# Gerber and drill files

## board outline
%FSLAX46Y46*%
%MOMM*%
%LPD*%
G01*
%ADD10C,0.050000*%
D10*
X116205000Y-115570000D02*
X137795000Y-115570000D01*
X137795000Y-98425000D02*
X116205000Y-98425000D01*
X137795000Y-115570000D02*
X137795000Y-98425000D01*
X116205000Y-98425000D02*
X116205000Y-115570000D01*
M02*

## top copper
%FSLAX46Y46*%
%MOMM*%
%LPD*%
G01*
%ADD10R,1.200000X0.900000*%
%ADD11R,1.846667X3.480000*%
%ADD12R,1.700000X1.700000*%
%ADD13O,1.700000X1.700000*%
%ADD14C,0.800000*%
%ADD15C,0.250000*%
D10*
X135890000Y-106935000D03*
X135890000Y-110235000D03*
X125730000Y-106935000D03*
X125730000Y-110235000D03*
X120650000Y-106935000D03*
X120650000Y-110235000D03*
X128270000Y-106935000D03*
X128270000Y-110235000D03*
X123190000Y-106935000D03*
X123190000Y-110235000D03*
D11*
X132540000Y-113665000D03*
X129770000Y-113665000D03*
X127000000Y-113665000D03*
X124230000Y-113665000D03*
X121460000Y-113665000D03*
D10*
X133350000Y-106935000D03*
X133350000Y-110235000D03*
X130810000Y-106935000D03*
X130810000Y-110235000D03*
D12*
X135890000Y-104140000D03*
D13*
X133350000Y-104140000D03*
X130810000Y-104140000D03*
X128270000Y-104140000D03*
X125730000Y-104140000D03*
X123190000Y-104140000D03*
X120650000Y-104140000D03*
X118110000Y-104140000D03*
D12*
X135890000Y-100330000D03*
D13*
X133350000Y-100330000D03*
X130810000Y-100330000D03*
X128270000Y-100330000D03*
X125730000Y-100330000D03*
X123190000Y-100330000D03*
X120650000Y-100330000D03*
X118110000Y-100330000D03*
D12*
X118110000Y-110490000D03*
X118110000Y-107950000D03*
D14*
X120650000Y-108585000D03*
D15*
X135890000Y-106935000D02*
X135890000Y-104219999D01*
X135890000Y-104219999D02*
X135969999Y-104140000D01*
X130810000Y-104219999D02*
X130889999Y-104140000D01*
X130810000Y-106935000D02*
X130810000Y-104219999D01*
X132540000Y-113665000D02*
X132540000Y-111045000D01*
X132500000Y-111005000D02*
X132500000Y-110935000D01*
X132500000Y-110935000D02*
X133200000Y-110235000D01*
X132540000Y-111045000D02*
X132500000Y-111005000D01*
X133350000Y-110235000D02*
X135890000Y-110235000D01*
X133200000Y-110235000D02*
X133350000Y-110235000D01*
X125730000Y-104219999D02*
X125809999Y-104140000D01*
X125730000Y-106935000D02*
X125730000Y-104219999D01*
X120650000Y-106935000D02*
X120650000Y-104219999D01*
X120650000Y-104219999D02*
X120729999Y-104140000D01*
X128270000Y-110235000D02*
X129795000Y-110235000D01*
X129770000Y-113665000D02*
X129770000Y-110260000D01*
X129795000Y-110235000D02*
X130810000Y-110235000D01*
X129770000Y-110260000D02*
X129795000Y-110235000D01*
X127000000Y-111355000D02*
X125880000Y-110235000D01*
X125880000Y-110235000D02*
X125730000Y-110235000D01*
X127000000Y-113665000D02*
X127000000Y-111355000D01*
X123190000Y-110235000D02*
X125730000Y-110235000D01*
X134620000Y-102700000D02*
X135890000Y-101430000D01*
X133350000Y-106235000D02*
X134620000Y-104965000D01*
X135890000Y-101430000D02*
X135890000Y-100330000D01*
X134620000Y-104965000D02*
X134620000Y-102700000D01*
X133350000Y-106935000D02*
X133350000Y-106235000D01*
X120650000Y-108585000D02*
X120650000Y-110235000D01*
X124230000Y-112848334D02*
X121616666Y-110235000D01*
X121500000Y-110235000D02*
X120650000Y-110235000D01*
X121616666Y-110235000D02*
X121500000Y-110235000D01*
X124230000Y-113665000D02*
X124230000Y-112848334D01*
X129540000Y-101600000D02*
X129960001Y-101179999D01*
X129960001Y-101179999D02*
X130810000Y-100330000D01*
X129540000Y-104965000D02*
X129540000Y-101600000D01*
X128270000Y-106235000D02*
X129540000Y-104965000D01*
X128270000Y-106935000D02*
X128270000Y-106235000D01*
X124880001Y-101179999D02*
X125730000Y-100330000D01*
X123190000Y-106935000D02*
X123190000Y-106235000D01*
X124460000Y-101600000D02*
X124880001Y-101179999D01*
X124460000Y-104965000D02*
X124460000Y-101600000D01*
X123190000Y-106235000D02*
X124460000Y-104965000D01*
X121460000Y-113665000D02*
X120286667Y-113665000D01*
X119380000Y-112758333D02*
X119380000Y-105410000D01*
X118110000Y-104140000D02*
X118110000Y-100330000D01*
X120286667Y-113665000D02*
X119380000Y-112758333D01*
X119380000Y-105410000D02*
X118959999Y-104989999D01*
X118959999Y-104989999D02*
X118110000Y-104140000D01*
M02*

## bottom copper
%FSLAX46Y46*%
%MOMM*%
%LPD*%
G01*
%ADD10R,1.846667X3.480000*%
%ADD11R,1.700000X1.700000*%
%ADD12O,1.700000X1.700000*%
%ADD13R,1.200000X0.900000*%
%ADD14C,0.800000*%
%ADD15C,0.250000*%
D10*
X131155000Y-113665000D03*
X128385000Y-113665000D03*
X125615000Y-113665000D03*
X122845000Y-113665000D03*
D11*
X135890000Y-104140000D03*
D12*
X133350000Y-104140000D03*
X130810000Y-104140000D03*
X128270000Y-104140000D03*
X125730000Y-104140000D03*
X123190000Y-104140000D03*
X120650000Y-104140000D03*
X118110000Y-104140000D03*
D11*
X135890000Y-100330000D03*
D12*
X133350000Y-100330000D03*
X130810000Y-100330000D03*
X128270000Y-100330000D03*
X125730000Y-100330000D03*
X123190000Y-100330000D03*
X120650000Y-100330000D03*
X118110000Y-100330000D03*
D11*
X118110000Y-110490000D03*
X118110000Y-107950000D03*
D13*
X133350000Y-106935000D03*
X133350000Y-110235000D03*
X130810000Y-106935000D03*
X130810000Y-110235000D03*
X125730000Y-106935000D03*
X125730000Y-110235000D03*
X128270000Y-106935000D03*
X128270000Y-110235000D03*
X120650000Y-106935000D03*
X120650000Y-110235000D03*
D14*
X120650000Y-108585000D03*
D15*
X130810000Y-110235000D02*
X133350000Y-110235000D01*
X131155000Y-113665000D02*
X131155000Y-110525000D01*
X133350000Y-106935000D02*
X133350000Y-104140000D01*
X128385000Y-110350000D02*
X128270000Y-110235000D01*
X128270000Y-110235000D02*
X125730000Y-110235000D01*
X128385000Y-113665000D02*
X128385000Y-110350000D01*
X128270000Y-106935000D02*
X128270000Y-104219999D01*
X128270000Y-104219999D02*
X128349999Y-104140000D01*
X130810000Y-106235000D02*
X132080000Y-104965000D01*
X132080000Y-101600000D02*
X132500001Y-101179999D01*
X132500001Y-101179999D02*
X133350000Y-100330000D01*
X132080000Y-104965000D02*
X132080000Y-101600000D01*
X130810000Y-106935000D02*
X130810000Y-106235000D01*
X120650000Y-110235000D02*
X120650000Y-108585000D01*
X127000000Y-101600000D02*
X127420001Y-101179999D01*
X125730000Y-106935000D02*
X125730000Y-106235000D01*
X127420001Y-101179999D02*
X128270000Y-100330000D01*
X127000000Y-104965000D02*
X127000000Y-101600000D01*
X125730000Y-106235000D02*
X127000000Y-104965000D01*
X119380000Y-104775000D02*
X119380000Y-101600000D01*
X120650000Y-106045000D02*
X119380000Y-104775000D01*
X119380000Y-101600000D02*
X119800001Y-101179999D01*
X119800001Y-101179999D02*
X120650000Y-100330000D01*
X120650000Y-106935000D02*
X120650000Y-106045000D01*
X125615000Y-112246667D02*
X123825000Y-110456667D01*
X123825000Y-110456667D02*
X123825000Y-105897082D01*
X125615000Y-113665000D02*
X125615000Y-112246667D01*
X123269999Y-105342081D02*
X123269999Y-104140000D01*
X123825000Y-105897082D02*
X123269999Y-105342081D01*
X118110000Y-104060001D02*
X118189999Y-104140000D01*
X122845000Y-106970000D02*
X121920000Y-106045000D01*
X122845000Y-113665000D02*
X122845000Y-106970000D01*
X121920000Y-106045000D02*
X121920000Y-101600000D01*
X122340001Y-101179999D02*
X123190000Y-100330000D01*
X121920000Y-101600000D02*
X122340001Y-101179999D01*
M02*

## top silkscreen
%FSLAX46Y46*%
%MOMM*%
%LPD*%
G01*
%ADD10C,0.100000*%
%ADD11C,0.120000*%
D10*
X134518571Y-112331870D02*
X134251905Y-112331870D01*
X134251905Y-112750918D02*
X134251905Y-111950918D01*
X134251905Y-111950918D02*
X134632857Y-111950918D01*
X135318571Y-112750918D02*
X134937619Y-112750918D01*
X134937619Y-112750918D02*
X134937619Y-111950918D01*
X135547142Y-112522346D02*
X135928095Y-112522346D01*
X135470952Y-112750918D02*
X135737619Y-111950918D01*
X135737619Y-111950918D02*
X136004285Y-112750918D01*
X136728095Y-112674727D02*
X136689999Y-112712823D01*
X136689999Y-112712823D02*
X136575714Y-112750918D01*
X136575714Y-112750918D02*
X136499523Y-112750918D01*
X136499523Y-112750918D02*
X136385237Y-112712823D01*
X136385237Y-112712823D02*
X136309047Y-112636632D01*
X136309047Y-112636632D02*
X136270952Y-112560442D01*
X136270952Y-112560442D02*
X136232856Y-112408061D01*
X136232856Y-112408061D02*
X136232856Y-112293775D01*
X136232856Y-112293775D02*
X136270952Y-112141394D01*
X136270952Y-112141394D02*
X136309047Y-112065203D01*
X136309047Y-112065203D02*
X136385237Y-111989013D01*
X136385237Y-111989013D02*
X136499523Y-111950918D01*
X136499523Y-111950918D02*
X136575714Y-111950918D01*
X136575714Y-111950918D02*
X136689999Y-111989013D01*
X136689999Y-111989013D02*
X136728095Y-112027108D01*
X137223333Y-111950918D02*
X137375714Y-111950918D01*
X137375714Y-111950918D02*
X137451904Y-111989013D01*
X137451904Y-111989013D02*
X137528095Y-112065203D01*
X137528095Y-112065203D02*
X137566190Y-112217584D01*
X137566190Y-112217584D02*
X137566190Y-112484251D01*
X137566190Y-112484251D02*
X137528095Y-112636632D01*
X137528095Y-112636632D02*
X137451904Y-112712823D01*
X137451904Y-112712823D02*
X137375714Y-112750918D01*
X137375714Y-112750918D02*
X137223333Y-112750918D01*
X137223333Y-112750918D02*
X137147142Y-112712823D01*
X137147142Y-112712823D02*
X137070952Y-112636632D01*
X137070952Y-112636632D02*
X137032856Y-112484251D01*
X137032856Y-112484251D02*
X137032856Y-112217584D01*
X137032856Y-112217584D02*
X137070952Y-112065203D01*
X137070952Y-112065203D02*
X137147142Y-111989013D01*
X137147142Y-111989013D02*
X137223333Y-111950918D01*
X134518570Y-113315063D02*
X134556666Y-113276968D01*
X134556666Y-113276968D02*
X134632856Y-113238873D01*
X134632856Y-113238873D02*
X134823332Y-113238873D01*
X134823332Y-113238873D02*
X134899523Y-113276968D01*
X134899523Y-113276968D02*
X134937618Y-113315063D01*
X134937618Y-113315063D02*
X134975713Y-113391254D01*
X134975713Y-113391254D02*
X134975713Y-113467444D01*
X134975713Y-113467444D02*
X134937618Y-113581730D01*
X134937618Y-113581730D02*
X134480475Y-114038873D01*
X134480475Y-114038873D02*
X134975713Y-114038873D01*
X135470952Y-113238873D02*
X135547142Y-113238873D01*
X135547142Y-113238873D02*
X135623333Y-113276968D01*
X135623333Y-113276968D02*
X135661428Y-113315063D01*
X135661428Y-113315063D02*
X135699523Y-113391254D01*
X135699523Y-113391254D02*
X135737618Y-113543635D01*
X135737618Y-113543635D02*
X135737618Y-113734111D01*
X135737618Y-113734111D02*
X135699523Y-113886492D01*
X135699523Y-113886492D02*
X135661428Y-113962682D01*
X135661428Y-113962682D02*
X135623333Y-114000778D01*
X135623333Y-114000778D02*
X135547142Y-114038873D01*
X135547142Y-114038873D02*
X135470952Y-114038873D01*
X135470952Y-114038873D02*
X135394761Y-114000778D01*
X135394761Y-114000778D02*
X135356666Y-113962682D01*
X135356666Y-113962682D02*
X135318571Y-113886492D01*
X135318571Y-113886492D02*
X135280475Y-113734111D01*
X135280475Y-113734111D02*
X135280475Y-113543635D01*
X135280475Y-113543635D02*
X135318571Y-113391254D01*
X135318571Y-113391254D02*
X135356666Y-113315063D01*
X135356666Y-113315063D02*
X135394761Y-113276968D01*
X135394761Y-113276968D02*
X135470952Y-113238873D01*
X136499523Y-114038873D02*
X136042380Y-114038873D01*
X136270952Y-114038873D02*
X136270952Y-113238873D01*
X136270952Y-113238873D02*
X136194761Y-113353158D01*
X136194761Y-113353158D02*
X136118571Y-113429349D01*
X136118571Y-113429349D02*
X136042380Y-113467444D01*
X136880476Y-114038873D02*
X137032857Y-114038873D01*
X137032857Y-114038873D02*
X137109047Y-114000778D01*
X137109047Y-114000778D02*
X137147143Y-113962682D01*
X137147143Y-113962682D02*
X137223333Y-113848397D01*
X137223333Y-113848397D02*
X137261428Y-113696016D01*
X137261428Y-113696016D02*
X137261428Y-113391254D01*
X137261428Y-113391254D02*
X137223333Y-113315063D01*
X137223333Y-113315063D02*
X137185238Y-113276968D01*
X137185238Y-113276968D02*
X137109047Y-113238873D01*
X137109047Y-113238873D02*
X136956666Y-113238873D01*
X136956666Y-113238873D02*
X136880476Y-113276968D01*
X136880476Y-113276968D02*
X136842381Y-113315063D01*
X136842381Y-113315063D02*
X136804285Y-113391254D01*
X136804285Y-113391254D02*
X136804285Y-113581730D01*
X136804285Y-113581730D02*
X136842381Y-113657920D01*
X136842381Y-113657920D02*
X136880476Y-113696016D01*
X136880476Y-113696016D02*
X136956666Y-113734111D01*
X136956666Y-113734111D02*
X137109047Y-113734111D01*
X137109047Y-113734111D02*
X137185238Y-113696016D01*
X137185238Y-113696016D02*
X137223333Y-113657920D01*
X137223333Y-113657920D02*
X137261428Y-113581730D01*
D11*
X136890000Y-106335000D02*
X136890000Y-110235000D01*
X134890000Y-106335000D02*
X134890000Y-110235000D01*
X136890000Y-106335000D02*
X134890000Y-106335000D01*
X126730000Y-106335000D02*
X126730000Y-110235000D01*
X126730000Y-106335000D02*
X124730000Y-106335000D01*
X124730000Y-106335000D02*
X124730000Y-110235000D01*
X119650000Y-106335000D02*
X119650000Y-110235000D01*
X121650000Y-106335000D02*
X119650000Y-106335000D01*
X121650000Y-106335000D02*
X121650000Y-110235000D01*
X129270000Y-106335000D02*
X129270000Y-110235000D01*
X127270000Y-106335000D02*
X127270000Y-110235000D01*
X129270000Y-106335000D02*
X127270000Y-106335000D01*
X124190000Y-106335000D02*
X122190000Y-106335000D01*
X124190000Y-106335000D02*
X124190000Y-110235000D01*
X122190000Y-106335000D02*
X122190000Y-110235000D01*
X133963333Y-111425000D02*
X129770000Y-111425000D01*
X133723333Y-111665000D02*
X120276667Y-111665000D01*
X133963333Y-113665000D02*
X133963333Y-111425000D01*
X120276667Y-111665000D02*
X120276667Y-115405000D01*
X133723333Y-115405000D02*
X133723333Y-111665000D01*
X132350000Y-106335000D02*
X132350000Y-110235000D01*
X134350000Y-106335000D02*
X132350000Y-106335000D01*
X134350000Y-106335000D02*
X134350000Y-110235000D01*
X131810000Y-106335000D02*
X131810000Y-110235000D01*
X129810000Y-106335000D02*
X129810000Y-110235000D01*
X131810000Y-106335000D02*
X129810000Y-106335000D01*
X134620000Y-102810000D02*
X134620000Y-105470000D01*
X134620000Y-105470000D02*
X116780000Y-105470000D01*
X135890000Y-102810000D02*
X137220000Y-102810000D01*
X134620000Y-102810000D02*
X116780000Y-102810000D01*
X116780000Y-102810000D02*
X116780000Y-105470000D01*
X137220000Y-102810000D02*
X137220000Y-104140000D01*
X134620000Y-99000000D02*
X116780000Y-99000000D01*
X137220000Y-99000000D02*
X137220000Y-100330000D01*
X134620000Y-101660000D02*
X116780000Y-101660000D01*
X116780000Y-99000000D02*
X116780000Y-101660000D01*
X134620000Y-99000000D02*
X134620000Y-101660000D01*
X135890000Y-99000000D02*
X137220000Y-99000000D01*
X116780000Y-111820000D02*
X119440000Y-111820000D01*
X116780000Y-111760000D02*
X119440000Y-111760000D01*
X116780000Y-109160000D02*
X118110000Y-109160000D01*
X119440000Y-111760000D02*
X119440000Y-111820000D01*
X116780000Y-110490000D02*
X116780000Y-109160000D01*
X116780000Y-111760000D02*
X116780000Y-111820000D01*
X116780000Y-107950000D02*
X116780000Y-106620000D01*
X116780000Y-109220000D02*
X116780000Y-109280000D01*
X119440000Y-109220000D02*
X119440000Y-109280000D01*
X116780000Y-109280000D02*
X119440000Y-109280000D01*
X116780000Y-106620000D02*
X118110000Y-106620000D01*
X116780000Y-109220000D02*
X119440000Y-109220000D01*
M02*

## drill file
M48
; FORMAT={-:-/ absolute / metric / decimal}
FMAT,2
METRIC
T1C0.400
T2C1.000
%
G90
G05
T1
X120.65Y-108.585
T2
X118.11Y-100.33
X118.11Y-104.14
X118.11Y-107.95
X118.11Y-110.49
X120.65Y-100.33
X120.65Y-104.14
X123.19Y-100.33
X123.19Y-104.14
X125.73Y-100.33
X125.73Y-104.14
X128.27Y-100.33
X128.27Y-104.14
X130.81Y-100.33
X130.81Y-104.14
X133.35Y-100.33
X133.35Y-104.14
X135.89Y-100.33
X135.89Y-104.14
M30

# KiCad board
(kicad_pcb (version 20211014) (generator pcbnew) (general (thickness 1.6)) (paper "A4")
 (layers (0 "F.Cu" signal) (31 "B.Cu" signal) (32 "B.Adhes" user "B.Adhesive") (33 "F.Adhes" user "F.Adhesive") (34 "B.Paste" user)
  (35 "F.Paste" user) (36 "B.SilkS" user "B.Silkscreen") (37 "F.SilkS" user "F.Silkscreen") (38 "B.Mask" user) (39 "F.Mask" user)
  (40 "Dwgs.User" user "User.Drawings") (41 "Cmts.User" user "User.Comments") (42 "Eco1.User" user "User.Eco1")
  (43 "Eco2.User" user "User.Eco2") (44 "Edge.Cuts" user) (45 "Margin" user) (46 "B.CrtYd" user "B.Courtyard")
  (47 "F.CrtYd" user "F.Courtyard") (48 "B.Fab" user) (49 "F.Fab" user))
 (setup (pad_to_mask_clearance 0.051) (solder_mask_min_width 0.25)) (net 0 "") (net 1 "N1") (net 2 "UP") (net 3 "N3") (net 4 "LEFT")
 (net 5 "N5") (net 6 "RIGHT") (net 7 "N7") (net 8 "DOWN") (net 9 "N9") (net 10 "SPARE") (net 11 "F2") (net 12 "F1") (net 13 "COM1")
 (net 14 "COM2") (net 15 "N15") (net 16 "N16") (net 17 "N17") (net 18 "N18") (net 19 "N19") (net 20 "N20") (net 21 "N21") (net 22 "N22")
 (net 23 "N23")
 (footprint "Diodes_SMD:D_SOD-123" (layer "F.Cu") (at 135.89 108.585 -90) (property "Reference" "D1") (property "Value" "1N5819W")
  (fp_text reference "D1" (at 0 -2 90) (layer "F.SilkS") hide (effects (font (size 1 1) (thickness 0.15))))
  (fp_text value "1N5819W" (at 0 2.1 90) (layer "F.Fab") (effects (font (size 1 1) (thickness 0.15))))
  (fp_line (start -2.25 -1) (end 1.65 -1) (layer "F.SilkS") (width 0.12))
  (fp_line (start -2.25 1) (end 1.65 1) (layer "F.SilkS") (width 0.12))
  (fp_line (start -2.25 -1) (end -2.25 1) (layer "F.SilkS") (width 0.12))
  (pad "1" smd rect locked (at -1.65 0 270) (size 0.9 1.2) (layers "F.Cu" "F.Paste" "F.Mask") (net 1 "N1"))
  (pad "2" smd rect locked (at 1.65 0 270) (size 0.9 1.2) (layers "F.Cu" "F.Paste" "F.Mask") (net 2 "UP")))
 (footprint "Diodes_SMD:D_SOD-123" (layer "F.Cu") (at 125.73 108.585 -90) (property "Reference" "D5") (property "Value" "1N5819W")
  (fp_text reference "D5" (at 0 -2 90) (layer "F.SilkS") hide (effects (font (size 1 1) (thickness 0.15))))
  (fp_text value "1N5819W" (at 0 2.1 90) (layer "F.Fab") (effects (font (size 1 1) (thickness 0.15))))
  (fp_line (start -2.25 -1) (end 1.65 -1) (layer "F.SilkS") (width 0.12))
  (fp_line (start -2.25 -1) (end -2.25 1) (layer "F.SilkS") (width 0.12))
  (fp_line (start -2.25 1) (end 1.65 1) (layer "F.SilkS") (width 0.12))
  (pad "1" smd rect locked (at -1.65 0 270) (size 0.9 1.2) (layers "F.Cu" "F.Paste" "F.Mask") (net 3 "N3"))
  (pad "2" smd rect locked (at 1.65 0 270) (size 0.9 1.2) (layers "F.Cu" "F.Paste" "F.Mask") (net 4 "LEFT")))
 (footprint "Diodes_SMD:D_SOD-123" (layer "F.Cu") (at 120.65 108.585 -90) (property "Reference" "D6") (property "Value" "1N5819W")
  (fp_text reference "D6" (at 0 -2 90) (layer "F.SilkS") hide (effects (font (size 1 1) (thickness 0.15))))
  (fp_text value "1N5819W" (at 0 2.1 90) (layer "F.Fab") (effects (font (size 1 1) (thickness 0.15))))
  (fp_line (start -2.25 1) (end 1.65 1) (layer "F.SilkS") (width 0.12))
  (fp_line (start -2.25 -1) (end -2.25 1) (layer "F.SilkS") (width 0.12))
  (fp_line (start -2.25 -1) (end 1.65 -1) (layer "F.SilkS") (width 0.12))
  (pad "1" smd rect locked (at -1.65 0 270) (size 0.9 1.2) (layers "F.Cu" "F.Paste" "F.Mask") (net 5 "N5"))
  (pad "2" smd rect locked (at 1.65 0 270) (size 0.9 1.2) (layers "F.Cu" "F.Paste" "F.Mask") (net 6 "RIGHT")))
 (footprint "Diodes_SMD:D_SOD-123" (layer "F.Cu") (at 128.27 108.585 -90) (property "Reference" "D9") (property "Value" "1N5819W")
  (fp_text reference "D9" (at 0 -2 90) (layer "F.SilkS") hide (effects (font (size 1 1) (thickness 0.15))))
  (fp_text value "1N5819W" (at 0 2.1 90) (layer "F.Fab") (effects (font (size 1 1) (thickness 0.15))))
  (fp_line (start -2.25 -1) (end 1.65 -1) (layer "F.SilkS") (width 0.12))
  (fp_line (start -2.25 1) (end 1.65 1) (layer "F.SilkS") (width 0.12))
  (fp_line (start -2.25 -1) (end -2.25 1) (layer "F.SilkS") (width 0.12))
  (pad "1" smd rect locked (at -1.65 0 270) (size 0.9 1.2) (layers "F.Cu" "F.Paste" "F.Mask") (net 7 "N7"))
  (pad "2" smd rect locked (at 1.65 0 270) (size 0.9 1.2) (layers "F.Cu" "F.Paste" "F.Mask") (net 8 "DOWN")))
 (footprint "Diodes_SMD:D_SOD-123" (layer "F.Cu") (at 123.19 108.585 -90) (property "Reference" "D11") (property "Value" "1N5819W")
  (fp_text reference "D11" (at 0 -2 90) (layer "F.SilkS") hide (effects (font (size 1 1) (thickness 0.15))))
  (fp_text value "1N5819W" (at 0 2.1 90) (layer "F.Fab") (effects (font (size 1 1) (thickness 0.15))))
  (fp_line (start -2.25 -1) (end -2.25 1) (layer "F.SilkS") (width 0.12))
  (fp_line (start -2.25 -1) (end 1.65 -1) (layer "F.SilkS") (width 0.12))
  (fp_line (start -2.25 1) (end 1.65 1) (layer "F.SilkS") (width 0.12))
  (pad "1" smd rect locked (at -1.65 0 270) (size 0.9 1.2) (layers "F.Cu" "F.Paste" "F.Mask") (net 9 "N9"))
  (pad "2" smd rect locked (at 1.65 0 270) (size 0.9 1.2) (layers "F.Cu" "F.Paste" "F.Mask") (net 4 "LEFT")))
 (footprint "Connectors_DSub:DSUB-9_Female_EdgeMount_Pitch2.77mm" (layer "F.Cu") (at 127 113.665) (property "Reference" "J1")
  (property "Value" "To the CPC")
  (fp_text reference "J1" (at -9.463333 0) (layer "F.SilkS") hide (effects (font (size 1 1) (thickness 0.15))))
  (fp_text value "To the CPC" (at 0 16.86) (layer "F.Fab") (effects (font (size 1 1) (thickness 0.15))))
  (fp_line (start 6.963333 -2.24) (end 2.77 -2.24) (layer "F.SilkS") (width 0.12))
  (fp_line (start 6.723333 -2) (end -6.723333 -2) (layer "F.SilkS") (width 0.12))
  (fp_line (start 6.963333 0) (end 6.963333 -2.24) (layer "F.SilkS") (width 0.12))
  (fp_line (start -6.723333 -2) (end -6.723333 1.74) (layer "F.SilkS") (width 0.12))
  (fp_line (start 6.723333 1.74) (end 6.723333 -2) (layer "F.SilkS") (width 0.12))
  (pad "1" smd rect locked (at 5.54 0) (size 1.846667 3.48) (layers "F.Cu" "F.Paste" "F.Mask") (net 2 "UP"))
  (pad "2" smd rect locked (at 2.77 0) (size 1.846667 3.48) (layers "F.Cu" "F.Paste" "F.Mask") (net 8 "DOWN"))
  (pad "3" smd rect locked (at 0 0) (size 1.846667 3.48) (layers "F.Cu" "F.Paste" "F.Mask") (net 4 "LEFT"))
  (pad "4" smd rect locked (at -2.77 0) (size 1.846667 3.48) (layers "F.Cu" "F.Paste" "F.Mask") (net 6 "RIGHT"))
  (pad "5" smd rect locked (at -5.54 0) (size 1.846667 3.48) (layers "F.Cu" "F.Paste" "F.Mask") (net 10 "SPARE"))
  (pad "6" smd rect locked (at 4.155 0) (size 1.846667 3.48) (layers "B.Cu" "B.Paste" "B.Mask") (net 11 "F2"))
  (pad "7" smd rect locked (at 1.385 0) (size 1.846667 3.48) (layers "B.Cu" "B.Paste" "B.Mask") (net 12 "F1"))
  (pad "8" smd rect locked (at -1.385 0) (size 1.846667 3.48) (layers "B.Cu" "B.Paste" "B.Mask") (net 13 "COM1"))
  (pad "9" smd rect locked (at -4.155 0) (size 1.846667 3.48) (layers "B.Cu" "B.Paste" "B.Mask") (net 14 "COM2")))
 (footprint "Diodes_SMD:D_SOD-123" (layer "F.Cu") (at 133.35 108.585 -90) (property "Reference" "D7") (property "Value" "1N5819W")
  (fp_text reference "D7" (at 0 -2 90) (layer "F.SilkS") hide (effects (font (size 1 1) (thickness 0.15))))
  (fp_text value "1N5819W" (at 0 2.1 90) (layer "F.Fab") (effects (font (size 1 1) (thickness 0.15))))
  (fp_line (start -2.25 1) (end 1.65 1) (layer "F.SilkS") (width 0.12))
  (fp_line (start -2.25 -1) (end -2.25 1) (layer "F.SilkS") (width 0.12))
  (fp_line (start -2.25 -1) (end 1.65 -1) (layer "F.SilkS") (width 0.12))
  (pad "1" smd rect locked (at -1.65 0 270) (size 0.9 1.2) (layers "F.Cu" "F.Paste" "F.Mask") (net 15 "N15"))
  (pad "2" smd rect locked (at 1.65 0 270) (size 0.9 1.2) (layers "F.Cu" "F.Paste" "F.Mask") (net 2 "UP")))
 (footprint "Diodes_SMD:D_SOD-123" (layer "F.Cu") (at 130.81 108.585 -90) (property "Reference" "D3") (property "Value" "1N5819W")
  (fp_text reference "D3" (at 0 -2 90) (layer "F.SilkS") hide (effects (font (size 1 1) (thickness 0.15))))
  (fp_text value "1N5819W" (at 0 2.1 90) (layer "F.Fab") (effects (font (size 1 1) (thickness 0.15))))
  (fp_line (start -2.25 -1) (end 1.65 -1) (layer "F.SilkS") (width 0.12))
  (fp_line (start -2.25 1) (end 1.65 1) (layer "F.SilkS") (width 0.12))
  (fp_line (start -2.25 -1) (end -2.25 1) (layer "F.SilkS") (width 0.12))
  (pad "1" smd rect locked (at -1.65 0 270) (size 0.9 1.2) (layers "F.Cu" "F.Paste" "F.Mask") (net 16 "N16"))
  (pad "2" smd rect locked (at 1.65 0 270) (size 0.9 1.2) (layers "F.Cu" "F.Paste" "F.Mask") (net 8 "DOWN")))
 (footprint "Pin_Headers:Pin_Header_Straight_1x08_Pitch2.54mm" (layer "F.Cu") (at 135.89 104.14 -90) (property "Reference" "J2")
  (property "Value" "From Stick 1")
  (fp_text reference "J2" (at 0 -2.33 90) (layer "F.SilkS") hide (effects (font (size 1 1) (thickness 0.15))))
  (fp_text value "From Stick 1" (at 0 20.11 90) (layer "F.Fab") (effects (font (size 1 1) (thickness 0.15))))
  (fp_line (start -1.33 1.27) (end 1.33 1.27) (layer "F.SilkS") (width 0.12))
  (fp_line (start 1.33 1.27) (end 1.33 19.11) (layer "F.SilkS") (width 0.12))
  (fp_line (start -1.33 0) (end -1.33 -1.33) (layer "F.SilkS") (width 0.12))
  (fp_line (start -1.33 1.27) (end -1.33 19.11) (layer "F.SilkS") (width 0.12))
  (fp_line (start -1.33 19.11) (end 1.33 19.11) (layer "F.SilkS") (width 0.12))
  (fp_line (start -1.33 -1.33) (end 0 -1.33) (layer "F.SilkS") (width 0.12))
  (pad "1" thru_hole rect locked (at 0 0 270) (size 1.7 1.7) (drill 1) (layers *.Cu *.Mask) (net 1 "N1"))
  (pad "2" thru_hole oval locked (at 0 2.54 270) (size 1.7 1.7) (drill 1) (layers *.Cu *.Mask) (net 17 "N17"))
  (pad "3" thru_hole oval locked (at 0 5.08 270) (size 1.7 1.7) (drill 1) (layers *.Cu *.Mask) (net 16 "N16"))
  (pad "4" thru_hole oval locked (at 0 7.62 270) (size 1.7 1.7) (drill 1) (layers *.Cu *.Mask) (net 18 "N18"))
  (pad "5" thru_hole oval locked (at 0 10.16 270) (size 1.7 1.7) (drill 1) (layers *.Cu *.Mask) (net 3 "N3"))
  (pad "6" thru_hole oval locked (at 0 12.7 270) (size 1.7 1.7) (drill 1) (layers *.Cu *.Mask) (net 13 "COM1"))
  (pad "7" thru_hole oval locked (at 0 15.24 270) (size 1.7 1.7) (drill 1) (layers *.Cu *.Mask) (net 5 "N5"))
  (pad "8" thru_hole oval locked (at 0 17.78 270) (size 1.7 1.7) (drill 1) (layers *.Cu *.Mask) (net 10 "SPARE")))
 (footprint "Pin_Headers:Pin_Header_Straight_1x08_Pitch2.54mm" (layer "F.Cu") (at 135.89 100.33 -90) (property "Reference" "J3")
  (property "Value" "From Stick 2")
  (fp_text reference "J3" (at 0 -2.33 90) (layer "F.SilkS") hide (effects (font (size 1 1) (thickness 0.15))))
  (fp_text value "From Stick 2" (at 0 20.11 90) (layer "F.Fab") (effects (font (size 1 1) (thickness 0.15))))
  (fp_line (start -1.33 1.27) (end -1.33 19.11) (layer "F.SilkS") (width 0.12))
  (fp_line (start -1.33 -1.33) (end 0 -1.33) (layer "F.SilkS") (width 0.12))
  (fp_line (start 1.33 1.27) (end 1.33 19.11) (layer "F.SilkS") (width 0.12))
  (fp_line (start -1.33 19.11) (end 1.33 19.11) (layer "F.SilkS") (width 0.12))
  (fp_line (start -1.33 1.27) (end 1.33 1.27) (layer "F.SilkS") (width 0.12))
  (fp_line (start -1.33 0) (end -1.33 -1.33) (layer "F.SilkS") (width 0.12))
  (pad "1" thru_hole rect locked (at 0 0 270) (size 1.7 1.7) (drill 1) (layers *.Cu *.Mask) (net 15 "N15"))
  (pad "2" thru_hole oval locked (at 0 2.54 270) (size 1.7 1.7) (drill 1) (layers *.Cu *.Mask) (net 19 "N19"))
  (pad "3" thru_hole oval locked (at 0 5.08 270) (size 1.7 1.7) (drill 1) (layers *.Cu *.Mask) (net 7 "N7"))
  (pad "4" thru_hole oval locked (at 0 7.62 270) (size 1.7 1.7) (drill 1) (layers *.Cu *.Mask) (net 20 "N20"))
  (pad "5" thru_hole oval locked (at 0 10.16 270) (size 1.7 1.7) (drill 1) (layers *.Cu *.Mask) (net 9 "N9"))
  (pad "6" thru_hole oval locked (at 0 12.7 270) (size 1.7 1.7) (drill 1) (layers *.Cu *.Mask) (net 14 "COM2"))
  (pad "7" thru_hole oval locked (at 0 15.24 270) (size 1.7 1.7) (drill 1) (layers *.Cu *.Mask) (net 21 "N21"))
  (pad "8" thru_hole oval locked (at 0 17.78 270) (size 1.7 1.7) (drill 1) (layers *.Cu *.Mask) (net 10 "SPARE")))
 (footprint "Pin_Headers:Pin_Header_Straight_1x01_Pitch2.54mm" (layer "F.Cu") (at 118.11 110.49) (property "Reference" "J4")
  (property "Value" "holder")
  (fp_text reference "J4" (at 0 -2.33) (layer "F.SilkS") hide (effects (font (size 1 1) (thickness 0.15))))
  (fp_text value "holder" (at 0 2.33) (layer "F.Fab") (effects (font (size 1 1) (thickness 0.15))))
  (fp_line (start -1.33 1.33) (end 1.33 1.33) (layer "F.SilkS") (width 0.12))
  (fp_line (start -1.33 1.27) (end 1.33 1.27) (layer "F.SilkS") (width 0.12))
  (fp_line (start -1.33 -1.33) (end 0 -1.33) (layer "F.SilkS") (width 0.12))
  (fp_line (start 1.33 1.27) (end 1.33 1.33) (layer "F.SilkS") (width 0.12))
  (fp_line (start -1.33 0) (end -1.33 -1.33) (layer "F.SilkS") (width 0.12))
  (fp_line (start -1.33 1.27) (end -1.33 1.33) (layer "F.SilkS") (width 0.12))
  (pad "1" thru_hole rect locked (at 0 0) (size 1.7 1.7) (drill 1) (layers *.Cu *.Mask) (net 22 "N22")))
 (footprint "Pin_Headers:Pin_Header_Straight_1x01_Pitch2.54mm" (layer "F.Cu") (at 118.11 107.95) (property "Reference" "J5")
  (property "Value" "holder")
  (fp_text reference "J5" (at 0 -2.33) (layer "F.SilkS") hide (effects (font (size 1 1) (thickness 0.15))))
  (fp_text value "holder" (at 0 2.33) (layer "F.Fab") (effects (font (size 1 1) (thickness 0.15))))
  (fp_line (start -1.33 0) (end -1.33 -1.33) (layer "F.SilkS") (width 0.12))
  (fp_line (start -1.33 1.27) (end -1.33 1.33) (layer "F.SilkS") (width 0.12))
  (fp_line (start 1.33 1.27) (end 1.33 1.33) (layer "F.SilkS") (width 0.12))
  (fp_line (start -1.33 1.33) (end 1.33 1.33) (layer "F.SilkS") (width 0.12))
  (fp_line (start -1.33 -1.33) (end 0 -1.33) (layer "F.SilkS") (width 0.12))
  (fp_line (start -1.33 1.27) (end 1.33 1.27) (layer "F.SilkS") (width 0.12))
  (pad "1" thru_hole rect locked (at 0 0) (size 1.7 1.7) (drill 1) (layers *.Cu *.Mask) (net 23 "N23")))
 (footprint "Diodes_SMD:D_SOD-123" (layer "B.Cu") (at 133.35 108.585 -90) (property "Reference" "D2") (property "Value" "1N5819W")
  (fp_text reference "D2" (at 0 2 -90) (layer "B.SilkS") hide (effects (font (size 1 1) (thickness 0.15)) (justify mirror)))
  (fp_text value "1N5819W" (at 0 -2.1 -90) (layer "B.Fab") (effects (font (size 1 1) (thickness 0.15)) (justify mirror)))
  (pad "1" smd rect locked (at -1.65 0 270) (size 0.9 1.2) (layers "B.Cu" "B.Paste" "B.Mask") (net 17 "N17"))
  (pad "2" smd rect locked (at 1.65 0 270) (size 0.9 1.2) (layers "B.Cu" "B.Paste" "B.Mask") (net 11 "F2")))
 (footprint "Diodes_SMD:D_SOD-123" (layer "B.Cu") (at 130.81 108.585 -90) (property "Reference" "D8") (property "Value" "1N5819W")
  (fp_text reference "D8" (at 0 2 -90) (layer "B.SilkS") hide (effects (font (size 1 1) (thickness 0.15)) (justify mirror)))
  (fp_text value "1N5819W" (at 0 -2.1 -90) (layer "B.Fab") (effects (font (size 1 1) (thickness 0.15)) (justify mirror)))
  (pad "1" smd rect locked (at -1.65 0 270) (size 0.9 1.2) (layers "B.Cu" "B.Paste" "B.Mask") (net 19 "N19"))
  (pad "2" smd rect locked (at 1.65 0 270) (size 0.9 1.2) (layers "B.Cu" "B.Paste" "B.Mask") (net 11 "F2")))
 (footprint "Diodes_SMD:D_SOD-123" (layer "B.Cu") (at 125.73 108.585 -90) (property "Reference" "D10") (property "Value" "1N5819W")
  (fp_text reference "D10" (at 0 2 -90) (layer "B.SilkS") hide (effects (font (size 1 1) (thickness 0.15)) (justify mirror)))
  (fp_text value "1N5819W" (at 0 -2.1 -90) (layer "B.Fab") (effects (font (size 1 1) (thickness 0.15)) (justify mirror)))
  (pad "1" smd rect locked (at -1.65 0 270) (size 0.9 1.2) (layers "B.Cu" "B.Paste" "B.Mask") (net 20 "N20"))
  (pad "2" smd rect locked (at 1.65 0 270) (size 0.9 1.2) (layers "B.Cu" "B.Paste" "B.Mask") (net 12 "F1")))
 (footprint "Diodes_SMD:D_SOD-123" (layer "B.Cu") (at 128.27 108.585 -90) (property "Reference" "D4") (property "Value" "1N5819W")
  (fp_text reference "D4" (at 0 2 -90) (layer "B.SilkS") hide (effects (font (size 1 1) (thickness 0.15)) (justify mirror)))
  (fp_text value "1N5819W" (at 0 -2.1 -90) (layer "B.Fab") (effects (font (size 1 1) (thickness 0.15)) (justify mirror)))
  (pad "1" smd rect locked (at -1.65 0 270) (size 0.9 1.2) (layers "B.Cu" "B.Paste" "B.Mask") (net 18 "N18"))
  (pad "2" smd rect locked (at 1.65 0 270) (size 0.9 1.2) (layers "B.Cu" "B.Paste" "B.Mask") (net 12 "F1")))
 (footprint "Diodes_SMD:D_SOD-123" (layer "B.Cu") (at 120.65 108.585 -90) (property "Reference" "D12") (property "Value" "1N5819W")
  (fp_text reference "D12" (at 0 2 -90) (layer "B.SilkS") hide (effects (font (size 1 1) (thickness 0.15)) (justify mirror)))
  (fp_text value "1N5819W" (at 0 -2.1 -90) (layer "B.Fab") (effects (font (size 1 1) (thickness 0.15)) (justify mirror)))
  (pad "1" smd rect locked (at -1.65 0 270) (size 0.9 1.2) (layers "B.Cu" "B.Paste" "B.Mask") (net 21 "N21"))
  (pad "2" smd rect locked (at 1.65 0 270) (size 0.9 1.2) (layers "B.Cu" "B.Paste" "B.Mask") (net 6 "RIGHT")))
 (gr_line (start 116.205 115.57) (end 137.795 115.57) (layer "Edge.Cuts") (width 0.05))
 (gr_line (start 137.795 98.425) (end 116.205 98.425) (layer "Edge.Cuts") (width 0.05))
 (gr_line (start 137.795 115.57) (end 137.795 98.425) (layer "Edge.Cuts") (width 0.05))
 (gr_line (start 116.205 98.425) (end 116.205 115.57) (layer "Edge.Cuts") (width 0.05))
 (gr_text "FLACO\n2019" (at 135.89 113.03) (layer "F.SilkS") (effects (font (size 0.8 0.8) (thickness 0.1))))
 (segment (start 130.81 110.235) (end 133.35 110.235) (width 0.25) (layer "B.Cu") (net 11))
 (segment (start 131.155 113.665) (end 131.155 110.525) (width 0.25) (layer "B.Cu") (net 11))
 (segment (start 135.89 106.935) (end 135.89 104.219999) (width 0.25) (layer "F.Cu") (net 1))
 (segment (start 135.89 104.219999) (end 135.969999 104.14) (width 0.25) (layer "F.Cu") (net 1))
 (segment (start 133.35 106.935) (end 133.35 104.14) (width 0.25) (layer "B.Cu") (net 17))
 (segment (start 128.385 110.35) (end 128.27 110.235) (width 0.25) (layer "B.Cu") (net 12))
 (segment (start 128.27 110.235) (end 125.73 110.235) (width 0.25) (layer "B.Cu") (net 12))
 (segment (start 128.385 113.665) (end 128.385 110.35) (width 0.25) (layer "B.Cu") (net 12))
 (segment (start 130.81 104.219999) (end 130.889999 104.14) (width 0.25) (layer "F.Cu") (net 16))
 (segment (start 130.81 106.935) (end 130.81 104.219999) (width 0.25) (layer "F.Cu") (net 16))
 (segment (start 128.27 106.935) (end 128.27 104.219999) (width 0.25) (layer "B.Cu") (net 18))
 (segment (start 128.27 104.219999) (end 128.349999 104.14) (width 0.25) (layer "B.Cu") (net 18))
 (segment (start 132.54 113.665) (end 132.54 111.045) (width 0.25) (layer "F.Cu") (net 2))
 (segment (start 132.5 111.005) (end 132.5 110.935) (width 0.25) (layer "F.Cu") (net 2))
 (segment (start 132.5 110.935) (end 133.2 110.235) (width 0.25) (layer "F.Cu") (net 2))
 (segment (start 132.54 111.045) (end 132.5 111.005) (width 0.25) (layer "F.Cu") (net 2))
 (segment (start 133.35 110.235) (end 135.89 110.235) (width 0.25) (layer "F.Cu") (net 2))
 (segment (start 133.2 110.235) (end 133.35 110.235) (width 0.25) (layer "F.Cu") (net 2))
 (segment (start 125.73 104.219999) (end 125.809999 104.14) (width 0.25) (layer "F.Cu") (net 3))
 (segment (start 125.73 106.935) (end 125.73 104.219999) (width 0.25) (layer "F.Cu") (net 3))
 (segment (start 120.65 106.935) (end 120.65 104.219999) (width 0.25) (layer "F.Cu") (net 5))
 (segment (start 120.65 104.219999) (end 120.729999 104.14) (width 0.25) (layer "F.Cu") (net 5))
 (segment (start 128.27 110.235) (end 129.795 110.235) (width 0.25) (layer "F.Cu") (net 8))
 (segment (start 129.77 113.665) (end 129.77 110.26) (width 0.25) (layer "F.Cu") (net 8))
 (segment (start 129.795 110.235) (end 130.81 110.235) (width 0.25) (layer "F.Cu") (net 8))
 (segment (start 129.77 110.26) (end 129.795 110.235) (width 0.25) (layer "F.Cu") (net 8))
 (segment (start 127 111.355) (end 125.88 110.235) (width 0.25) (layer "F.Cu") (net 4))
 (segment (start 125.88 110.235) (end 125.73 110.235) (width 0.25) (layer "F.Cu") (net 4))
 (segment (start 127 113.665) (end 127 111.355) (width 0.25) (layer "F.Cu") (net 4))
 (segment (start 123.19 110.235) (end 125.73 110.235) (width 0.25) (layer "F.Cu") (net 4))
 (segment (start 134.62 102.7) (end 135.89 101.43) (width 0.25) (layer "F.Cu") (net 15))
 (segment (start 133.35 106.235) (end 134.62 104.965) (width 0.25) (layer "F.Cu") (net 15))
 (segment (start 135.89 101.43) (end 135.89 100.33) (width 0.25) (layer "F.Cu") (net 15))
 (segment (start 134.62 104.965) (end 134.62 102.7) (width 0.25) (layer "F.Cu") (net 15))
 (segment (start 133.35 106.935) (end 133.35 106.235) (width 0.25) (layer "F.Cu") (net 15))
 (segment (start 130.81 106.235) (end 132.08 104.965) (width 0.25) (layer "B.Cu") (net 19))
 (segment (start 132.08 101.6) (end 132.500001 101.179999) (width 0.25) (layer "B.Cu") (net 19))
 (segment (start 132.500001 101.179999) (end 133.35 100.33) (width 0.25) (layer "B.Cu") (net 19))
 (segment (start 132.08 104.965) (end 132.08 101.6) (width 0.25) (layer "B.Cu") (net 19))
 (segment (start 130.81 106.935) (end 130.81 106.235) (width 0.25) (layer "B.Cu") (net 19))
 (segment (start 120.65 108.585) (end 120.65 110.235) (width 0.25) (layer "F.Cu") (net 6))
 (segment (start 124.23 112.848334) (end 121.616666 110.235) (width 0.25) (layer "F.Cu") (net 6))
 (segment (start 121.5 110.235) (end 120.65 110.235) (width 0.25) (layer "F.Cu") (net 6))
 (segment (start 121.616666 110.235) (end 121.5 110.235) (width 0.25) (layer "F.Cu") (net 6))
 (segment (start 124.23 113.665) (end 124.23 112.848334) (width 0.25) (layer "F.Cu") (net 6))
 (via (at 120.65 108.585) (size 0.8) (drill 0.4) (layers "F.Cu" "B.Cu") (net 6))
 (segment (start 120.65 110.235) (end 120.65 108.585) (width 0.25) (layer "B.Cu") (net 6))
 (segment (start 129.54 101.6) (end 129.960001 101.179999) (width 0.25) (layer "F.Cu") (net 7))
 (segment (start 129.960001 101.179999) (end 130.81 100.33) (width 0.25) (layer "F.Cu") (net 7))
 (segment (start 129.54 104.965) (end 129.54 101.6) (width 0.25) (layer "F.Cu") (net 7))
 (segment (start 128.27 106.235) (end 129.54 104.965) (width 0.25) (layer "F.Cu") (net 7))
 (segment (start 128.27 106.935) (end 128.27 106.235) (width 0.25) (layer "F.Cu") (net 7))
 (segment (start 127 101.6) (end 127.420001 101.179999) (width 0.25) (layer "B.Cu") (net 20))
 (segment (start 125.73 106.935) (end 125.73 106.235) (width 0.25) (layer "B.Cu") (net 20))
 (segment (start 127.420001 101.179999) (end 128.27 100.33) (width 0.25) (layer "B.Cu") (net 20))
 (segment (start 127 104.965) (end 127 101.6) (width 0.25) (layer "B.Cu") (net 20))
 (segment (start 125.73 106.235) (end 127 104.965) (width 0.25) (layer "B.Cu") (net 20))
 (segment (start 124.880001 101.179999) (end 125.73 100.33) (width 0.25) (layer "F.Cu") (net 9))
 (segment (start 123.19 106.935) (end 123.19 106.235) (width 0.25) (layer "F.Cu") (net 9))
 (segment (start 124.46 101.6) (end 124.880001 101.179999) (width 0.25) (layer "F.Cu") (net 9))
 (segment (start 124.46 104.965) (end 124.46 101.6) (width 0.25) (layer "F.Cu") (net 9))
 (segment (start 123.19 106.235) (end 124.46 104.965) (width 0.25) (layer "F.Cu") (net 9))
 (segment (start 119.38 104.775) (end 119.38 101.6) (width 0.25) (layer "B.Cu") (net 21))
 (segment (start 120.65 106.045) (end 119.38 104.775) (width 0.25) (layer "B.Cu") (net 21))
 (segment (start 119.38 101.6) (end 119.800001 101.179999) (width 0.25) (layer "B.Cu") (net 21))
 (segment (start 119.800001 101.179999) (end 120.65 100.33) (width 0.25) (layer "B.Cu") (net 21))
 (segment (start 120.65 106.935) (end 120.65 106.045) (width 0.25) (layer "B.Cu") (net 21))
 (segment (start 125.615 112.246667) (end 123.825 110.456667) (width 0.25) (layer "B.Cu") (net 13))
 (segment (start 123.825 110.456667) (end 123.825 105.897082) (width 0.25) (layer "B.Cu") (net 13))
 (segment (start 125.615 113.665) (end 125.615 112.246667) (width 0.25) (layer "B.Cu") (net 13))
 (segment (start 123.269999 105.342081) (end 123.269999 104.14) (width 0.25) (layer "B.Cu") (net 13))
 (segment (start 123.825 105.897082) (end 123.269999 105.342081) (width 0.25) (layer "B.Cu") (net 13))
 (segment (start 121.46 113.665) (end 120.286667 113.665) (width 0.25) (layer "F.Cu") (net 10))
 (segment (start 119.38 112.758333) (end 119.38 105.41) (width 0.25) (layer "F.Cu") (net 10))
 (segment (start 118.11 104.14) (end 118.11 100.33) (width 0.25) (layer "F.Cu") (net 10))
 (segment (start 120.286667 113.665) (end 119.38 112.758333) (width 0.25) (layer "F.Cu") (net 10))
 (segment (start 119.38 105.41) (end 118.959999 104.989999) (width 0.25) (layer "F.Cu") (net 10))
 (segment (start 118.959999 104.989999) (end 118.11 104.14) (width 0.25) (layer "F.Cu") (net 10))
 (segment (start 118.11 104.060001) (end 118.189999 104.14) (width 0.25) (layer "B.Cu") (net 10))
 (segment (start 122.845 106.97) (end 121.92 106.045) (width 0.25) (layer "B.Cu") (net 14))
 (segment (start 122.845 113.665) (end 122.845 106.97) (width 0.25) (layer "B.Cu") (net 14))
 (segment (start 121.92 106.045) (end 121.92 101.6) (width 0.25) (layer "B.Cu") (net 14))
 (segment (start 122.340001 101.179999) (end 123.19 100.33) (width 0.25) (layer "B.Cu") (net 14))
 (segment (start 121.92 101.6) (end 122.340001 101.179999) (width 0.25) (layer "B.Cu") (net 14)))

